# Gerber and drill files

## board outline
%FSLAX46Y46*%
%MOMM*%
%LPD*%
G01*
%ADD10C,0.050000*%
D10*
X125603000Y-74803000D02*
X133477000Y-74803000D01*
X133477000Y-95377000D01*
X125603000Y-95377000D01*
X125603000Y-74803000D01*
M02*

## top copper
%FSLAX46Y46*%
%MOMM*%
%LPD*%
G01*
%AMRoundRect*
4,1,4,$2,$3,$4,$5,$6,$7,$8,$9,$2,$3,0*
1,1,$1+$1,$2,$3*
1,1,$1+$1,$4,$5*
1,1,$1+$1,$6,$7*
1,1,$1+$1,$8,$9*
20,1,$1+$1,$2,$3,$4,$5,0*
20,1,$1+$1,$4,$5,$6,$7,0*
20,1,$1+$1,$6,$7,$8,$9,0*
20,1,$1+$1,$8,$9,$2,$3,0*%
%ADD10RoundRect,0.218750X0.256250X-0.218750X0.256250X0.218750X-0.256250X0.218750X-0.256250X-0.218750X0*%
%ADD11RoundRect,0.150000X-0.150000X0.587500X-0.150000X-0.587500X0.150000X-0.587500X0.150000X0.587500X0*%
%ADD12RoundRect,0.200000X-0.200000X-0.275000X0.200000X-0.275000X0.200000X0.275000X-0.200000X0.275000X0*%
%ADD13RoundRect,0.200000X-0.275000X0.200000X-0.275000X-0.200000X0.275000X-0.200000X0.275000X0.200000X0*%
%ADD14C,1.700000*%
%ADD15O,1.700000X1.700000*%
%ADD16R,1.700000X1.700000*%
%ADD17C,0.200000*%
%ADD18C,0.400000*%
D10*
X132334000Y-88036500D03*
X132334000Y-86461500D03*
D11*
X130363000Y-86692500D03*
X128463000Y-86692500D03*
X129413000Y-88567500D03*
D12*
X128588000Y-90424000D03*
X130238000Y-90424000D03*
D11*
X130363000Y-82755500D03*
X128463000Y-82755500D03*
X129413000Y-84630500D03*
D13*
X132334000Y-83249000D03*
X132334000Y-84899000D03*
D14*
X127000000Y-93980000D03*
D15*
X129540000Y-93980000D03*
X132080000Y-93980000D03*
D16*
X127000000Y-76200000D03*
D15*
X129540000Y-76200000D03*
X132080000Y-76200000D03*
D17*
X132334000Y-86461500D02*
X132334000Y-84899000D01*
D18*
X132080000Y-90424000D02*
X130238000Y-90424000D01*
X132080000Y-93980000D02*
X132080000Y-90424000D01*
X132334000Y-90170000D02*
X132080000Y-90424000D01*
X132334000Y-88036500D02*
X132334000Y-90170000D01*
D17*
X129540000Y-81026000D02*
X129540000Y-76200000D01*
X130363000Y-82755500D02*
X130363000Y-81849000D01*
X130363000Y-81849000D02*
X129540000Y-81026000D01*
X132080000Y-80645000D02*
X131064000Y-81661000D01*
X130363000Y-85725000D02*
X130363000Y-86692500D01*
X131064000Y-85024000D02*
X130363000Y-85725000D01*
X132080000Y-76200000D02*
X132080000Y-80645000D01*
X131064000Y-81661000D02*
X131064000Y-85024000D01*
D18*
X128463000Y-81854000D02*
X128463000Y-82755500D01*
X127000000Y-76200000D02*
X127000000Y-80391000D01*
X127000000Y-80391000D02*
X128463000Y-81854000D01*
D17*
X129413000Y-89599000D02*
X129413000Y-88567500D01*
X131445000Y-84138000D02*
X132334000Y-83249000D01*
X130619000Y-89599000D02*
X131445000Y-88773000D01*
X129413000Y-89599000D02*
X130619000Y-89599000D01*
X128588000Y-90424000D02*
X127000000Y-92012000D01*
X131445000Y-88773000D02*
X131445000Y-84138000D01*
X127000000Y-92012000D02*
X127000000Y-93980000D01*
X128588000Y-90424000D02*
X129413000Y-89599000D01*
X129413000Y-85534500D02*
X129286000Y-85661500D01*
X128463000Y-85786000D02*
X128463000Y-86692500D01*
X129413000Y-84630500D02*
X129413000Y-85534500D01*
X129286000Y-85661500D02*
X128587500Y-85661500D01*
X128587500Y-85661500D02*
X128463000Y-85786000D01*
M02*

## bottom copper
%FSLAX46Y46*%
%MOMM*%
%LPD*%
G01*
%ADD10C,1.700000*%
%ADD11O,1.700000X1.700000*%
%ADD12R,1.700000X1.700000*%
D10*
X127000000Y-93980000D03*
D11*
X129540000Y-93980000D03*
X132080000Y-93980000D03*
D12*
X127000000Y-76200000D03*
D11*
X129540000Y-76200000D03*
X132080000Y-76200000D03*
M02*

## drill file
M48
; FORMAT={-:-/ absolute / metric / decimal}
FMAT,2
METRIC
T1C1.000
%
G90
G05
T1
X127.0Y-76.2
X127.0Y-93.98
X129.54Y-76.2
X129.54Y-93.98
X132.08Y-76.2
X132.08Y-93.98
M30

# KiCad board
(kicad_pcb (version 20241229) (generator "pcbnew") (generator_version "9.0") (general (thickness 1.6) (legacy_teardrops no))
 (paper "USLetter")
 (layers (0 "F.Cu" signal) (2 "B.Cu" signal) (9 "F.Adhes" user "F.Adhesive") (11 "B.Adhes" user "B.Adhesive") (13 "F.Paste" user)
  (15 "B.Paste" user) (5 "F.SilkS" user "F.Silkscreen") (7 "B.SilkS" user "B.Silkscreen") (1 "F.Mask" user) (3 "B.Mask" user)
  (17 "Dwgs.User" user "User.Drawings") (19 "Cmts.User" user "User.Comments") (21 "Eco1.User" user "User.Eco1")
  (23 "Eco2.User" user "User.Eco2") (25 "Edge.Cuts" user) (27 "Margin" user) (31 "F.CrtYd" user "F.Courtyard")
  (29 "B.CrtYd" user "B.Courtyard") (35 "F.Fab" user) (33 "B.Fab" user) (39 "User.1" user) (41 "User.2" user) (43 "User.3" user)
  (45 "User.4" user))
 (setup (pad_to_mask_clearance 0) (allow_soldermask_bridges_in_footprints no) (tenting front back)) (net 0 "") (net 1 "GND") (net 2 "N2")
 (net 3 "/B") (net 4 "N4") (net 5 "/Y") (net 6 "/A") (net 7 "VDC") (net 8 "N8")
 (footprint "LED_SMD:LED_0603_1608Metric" (layer "F.Cu") (at 132.334 87.249 90)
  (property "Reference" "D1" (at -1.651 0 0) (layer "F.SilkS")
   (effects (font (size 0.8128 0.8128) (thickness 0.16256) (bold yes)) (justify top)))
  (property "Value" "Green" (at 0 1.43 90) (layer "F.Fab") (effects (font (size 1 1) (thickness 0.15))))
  (pad "1" smd roundrect (at -0.7875 0 90) (size 0.875 0.95) (layers "F.Cu" "F.Mask" "F.Paste") (roundrect_rratio 0.25) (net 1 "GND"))
  (pad "2" smd roundrect (at 0.7875 0 90) (size 0.875 0.95) (layers "F.Cu" "F.Mask" "F.Paste") (roundrect_rratio 0.25) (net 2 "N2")))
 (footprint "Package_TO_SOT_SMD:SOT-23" (layer "F.Cu") (at 129.413 87.63 -90)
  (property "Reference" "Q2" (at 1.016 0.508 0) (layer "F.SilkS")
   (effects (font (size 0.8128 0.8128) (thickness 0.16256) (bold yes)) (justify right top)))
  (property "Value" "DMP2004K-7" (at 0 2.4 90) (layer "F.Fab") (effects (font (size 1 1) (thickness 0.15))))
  (pad "1" smd roundrect (at -0.9375 -0.95 270) (size 1.475 0.6) (layers "F.Cu" "F.Mask" "F.Paste") (roundrect_rratio 0.25) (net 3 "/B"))
  (pad "2" smd roundrect (at -0.9375 0.95 270) (size 1.475 0.6) (layers "F.Cu" "F.Mask" "F.Paste") (roundrect_rratio 0.25) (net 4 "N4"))
  (pad "3" smd roundrect (at 0.9375 0 270) (size 1.475 0.6) (layers "F.Cu" "F.Mask" "F.Paste") (roundrect_rratio 0.25) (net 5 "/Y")))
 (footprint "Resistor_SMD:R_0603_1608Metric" (layer "F.Cu") (at 129.413 90.424)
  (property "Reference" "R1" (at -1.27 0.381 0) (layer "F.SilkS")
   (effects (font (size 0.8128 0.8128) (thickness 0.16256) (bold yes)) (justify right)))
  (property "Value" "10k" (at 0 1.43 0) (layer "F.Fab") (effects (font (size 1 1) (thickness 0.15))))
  (pad "1" smd roundrect (at -0.825 0) (size 0.8 0.95) (layers "F.Cu" "F.Mask" "F.Paste") (roundrect_rratio 0.25) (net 5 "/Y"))
  (pad "2" smd roundrect (at 0.825 0) (size 0.8 0.95) (layers "F.Cu" "F.Mask" "F.Paste") (roundrect_rratio 0.25) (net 1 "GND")))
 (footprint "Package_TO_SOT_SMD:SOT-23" (layer "F.Cu") (at 129.413 83.693 -90)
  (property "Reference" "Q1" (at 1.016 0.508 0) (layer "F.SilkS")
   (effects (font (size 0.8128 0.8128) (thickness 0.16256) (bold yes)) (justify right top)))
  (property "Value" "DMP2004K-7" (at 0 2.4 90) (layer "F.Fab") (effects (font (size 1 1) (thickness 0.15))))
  (pad "1" smd roundrect (at -0.9375 -0.95 270) (size 1.475 0.6) (layers "F.Cu" "F.Mask" "F.Paste") (roundrect_rratio 0.25) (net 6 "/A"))
  (pad "2" smd roundrect (at -0.9375 0.95 270) (size 1.475 0.6) (layers "F.Cu" "F.Mask" "F.Paste") (roundrect_rratio 0.25) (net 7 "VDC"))
  (pad "3" smd roundrect (at 0.9375 0 270) (size 1.475 0.6) (layers "F.Cu" "F.Mask" "F.Paste") (roundrect_rratio 0.25) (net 4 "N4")))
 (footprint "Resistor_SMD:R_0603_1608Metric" (layer "F.Cu") (at 132.334 84.074 -90)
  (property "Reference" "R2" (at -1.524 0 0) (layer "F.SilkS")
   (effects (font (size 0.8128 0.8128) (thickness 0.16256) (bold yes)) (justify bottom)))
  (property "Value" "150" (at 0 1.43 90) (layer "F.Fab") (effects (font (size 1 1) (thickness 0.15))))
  (pad "1" smd roundrect (at -0.825 0 270) (size 0.8 0.95) (layers "F.Cu" "F.Mask" "F.Paste") (roundrect_rratio 0.25) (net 5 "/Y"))
  (pad "2" smd roundrect (at 0.825 0 270) (size 0.8 0.95) (layers "F.Cu" "F.Mask" "F.Paste") (roundrect_rratio 0.25) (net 2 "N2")))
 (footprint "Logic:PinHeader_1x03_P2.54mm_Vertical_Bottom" (layer "B.Cu") (at 127 93.98 -90)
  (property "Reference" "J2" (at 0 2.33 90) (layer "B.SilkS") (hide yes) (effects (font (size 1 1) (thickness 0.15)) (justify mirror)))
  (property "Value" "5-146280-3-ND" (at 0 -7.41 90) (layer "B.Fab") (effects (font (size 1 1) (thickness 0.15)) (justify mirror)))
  (pad "1" thru_hole circle (at 0 0 270) (size 1.7 1.7) (drill 1) (layers "*.Cu" "*.Mask") (remove_unused_layers no) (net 5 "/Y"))
  (pad "2" thru_hole oval (at 0 -2.54 270) (size 1.7 1.7) (drill 1) (layers "*.Cu" "*.Mask") (remove_unused_layers no) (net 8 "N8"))
  (pad "3" thru_hole oval (at 0 -5.08 270) (size 1.7 1.7) (drill 1) (layers "*.Cu" "*.Mask") (remove_unused_layers no) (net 1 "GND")))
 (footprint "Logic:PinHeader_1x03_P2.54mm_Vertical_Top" (layer "B.Cu") (at 127 76.2 -90)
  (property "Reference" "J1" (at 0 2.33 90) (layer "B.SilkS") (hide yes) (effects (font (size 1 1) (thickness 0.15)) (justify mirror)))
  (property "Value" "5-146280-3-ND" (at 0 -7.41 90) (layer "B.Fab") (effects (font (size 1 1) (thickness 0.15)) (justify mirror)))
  (pad "1" thru_hole rect (at 0 0 270) (size 1.7 1.7) (drill 1) (layers "*.Cu" "*.Mask") (remove_unused_layers no) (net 7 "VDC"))
  (pad "2" thru_hole oval (at 0 -2.54 270) (size 1.7 1.7) (drill 1) (layers "*.Cu" "*.Mask") (remove_unused_layers no) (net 6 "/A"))
  (pad "3" thru_hole oval (at 0 -5.08 270) (size 1.7 1.7) (drill 1) (layers "*.Cu" "*.Mask") (remove_unused_layers no) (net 3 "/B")))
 (gr_rect (start 125.603 74.803) (end 133.477 95.377) (stroke (width 0.05) (type default)) (fill no) (layer "Edge.Cuts"))
 (segment (start 132.334 86.4615) (end 132.334 84.899) (width 0.2) (layer "F.Cu") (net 2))
 (segment (start 132.08 90.424) (end 130.238 90.424) (width 0.4) (layer "F.Cu") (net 1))
 (segment (start 132.08 93.98) (end 132.08 90.424) (width 0.4) (layer "F.Cu") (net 1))
 (segment (start 132.334 90.17) (end 132.08 90.424) (width 0.4) (layer "F.Cu") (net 1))
 (segment (start 132.334 88.0365) (end 132.334 90.17) (width 0.4) (layer "F.Cu") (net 1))
 (segment (start 129.54 81.026) (end 129.54 76.2) (width 0.2) (layer "F.Cu") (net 6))
 (segment (start 130.363 82.7555) (end 130.363 81.849) (width 0.2) (layer "F.Cu") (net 6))
 (segment (start 130.363 81.849) (end 129.54 81.026) (width 0.2) (layer "F.Cu") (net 6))
 (segment (start 132.08 80.645) (end 131.064 81.661) (width 0.2) (layer "F.Cu") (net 3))
 (segment (start 130.363 85.725) (end 130.363 86.6925) (width 0.2) (layer "F.Cu") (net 3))
 (segment (start 131.064 85.024) (end 130.363 85.725) (width 0.2) (layer "F.Cu") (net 3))
 (segment (start 132.08 76.2) (end 132.08 80.645) (width 0.2) (layer "F.Cu") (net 3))
 (segment (start 131.064 81.661) (end 131.064 85.024) (width 0.2) (layer "F.Cu") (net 3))
 (segment (start 128.463 81.854) (end 128.463 82.7555) (width 0.4) (layer "F.Cu") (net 7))
 (segment (start 127 76.2) (end 127 80.391) (width 0.4) (layer "F.Cu") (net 7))
 (segment (start 127 80.391) (end 128.463 81.854) (width 0.4) (layer "F.Cu") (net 7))
 (segment (start 129.413 89.599) (end 129.413 88.5675) (width 0.2) (layer "F.Cu") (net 5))
 (segment (start 131.445 84.138) (end 132.334 83.249) (width 0.2) (layer "F.Cu") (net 5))
 (segment (start 130.619 89.599) (end 131.445 88.773) (width 0.2) (layer "F.Cu") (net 5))
 (segment (start 129.413 89.599) (end 130.619 89.599) (width 0.2) (layer "F.Cu") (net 5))
 (segment (start 128.588 90.424) (end 127 92.012) (width 0.2) (layer "F.Cu") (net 5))
 (segment (start 131.445 88.773) (end 131.445 84.138) (width 0.2) (layer "F.Cu") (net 5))
 (segment (start 127 92.012) (end 127 93.98) (width 0.2) (layer "F.Cu") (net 5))
 (segment (start 128.588 90.424) (end 129.413 89.599) (width 0.2) (layer "F.Cu") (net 5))
 (segment (start 129.413 85.5345) (end 129.286 85.6615) (width 0.2) (layer "F.Cu") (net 4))
 (segment (start 128.463 85.786) (end 128.463 86.6925) (width 0.2) (layer "F.Cu") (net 4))
 (segment (start 129.413 84.6305) (end 129.413 85.5345) (width 0.2) (layer "F.Cu") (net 4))
 (segment (start 129.286 85.6615) (end 128.5875 85.6615) (width 0.2) (layer "F.Cu") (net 4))
 (segment (start 128.5875 85.6615) (end 128.463 85.786) (width 0.2) (layer "F.Cu") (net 4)))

